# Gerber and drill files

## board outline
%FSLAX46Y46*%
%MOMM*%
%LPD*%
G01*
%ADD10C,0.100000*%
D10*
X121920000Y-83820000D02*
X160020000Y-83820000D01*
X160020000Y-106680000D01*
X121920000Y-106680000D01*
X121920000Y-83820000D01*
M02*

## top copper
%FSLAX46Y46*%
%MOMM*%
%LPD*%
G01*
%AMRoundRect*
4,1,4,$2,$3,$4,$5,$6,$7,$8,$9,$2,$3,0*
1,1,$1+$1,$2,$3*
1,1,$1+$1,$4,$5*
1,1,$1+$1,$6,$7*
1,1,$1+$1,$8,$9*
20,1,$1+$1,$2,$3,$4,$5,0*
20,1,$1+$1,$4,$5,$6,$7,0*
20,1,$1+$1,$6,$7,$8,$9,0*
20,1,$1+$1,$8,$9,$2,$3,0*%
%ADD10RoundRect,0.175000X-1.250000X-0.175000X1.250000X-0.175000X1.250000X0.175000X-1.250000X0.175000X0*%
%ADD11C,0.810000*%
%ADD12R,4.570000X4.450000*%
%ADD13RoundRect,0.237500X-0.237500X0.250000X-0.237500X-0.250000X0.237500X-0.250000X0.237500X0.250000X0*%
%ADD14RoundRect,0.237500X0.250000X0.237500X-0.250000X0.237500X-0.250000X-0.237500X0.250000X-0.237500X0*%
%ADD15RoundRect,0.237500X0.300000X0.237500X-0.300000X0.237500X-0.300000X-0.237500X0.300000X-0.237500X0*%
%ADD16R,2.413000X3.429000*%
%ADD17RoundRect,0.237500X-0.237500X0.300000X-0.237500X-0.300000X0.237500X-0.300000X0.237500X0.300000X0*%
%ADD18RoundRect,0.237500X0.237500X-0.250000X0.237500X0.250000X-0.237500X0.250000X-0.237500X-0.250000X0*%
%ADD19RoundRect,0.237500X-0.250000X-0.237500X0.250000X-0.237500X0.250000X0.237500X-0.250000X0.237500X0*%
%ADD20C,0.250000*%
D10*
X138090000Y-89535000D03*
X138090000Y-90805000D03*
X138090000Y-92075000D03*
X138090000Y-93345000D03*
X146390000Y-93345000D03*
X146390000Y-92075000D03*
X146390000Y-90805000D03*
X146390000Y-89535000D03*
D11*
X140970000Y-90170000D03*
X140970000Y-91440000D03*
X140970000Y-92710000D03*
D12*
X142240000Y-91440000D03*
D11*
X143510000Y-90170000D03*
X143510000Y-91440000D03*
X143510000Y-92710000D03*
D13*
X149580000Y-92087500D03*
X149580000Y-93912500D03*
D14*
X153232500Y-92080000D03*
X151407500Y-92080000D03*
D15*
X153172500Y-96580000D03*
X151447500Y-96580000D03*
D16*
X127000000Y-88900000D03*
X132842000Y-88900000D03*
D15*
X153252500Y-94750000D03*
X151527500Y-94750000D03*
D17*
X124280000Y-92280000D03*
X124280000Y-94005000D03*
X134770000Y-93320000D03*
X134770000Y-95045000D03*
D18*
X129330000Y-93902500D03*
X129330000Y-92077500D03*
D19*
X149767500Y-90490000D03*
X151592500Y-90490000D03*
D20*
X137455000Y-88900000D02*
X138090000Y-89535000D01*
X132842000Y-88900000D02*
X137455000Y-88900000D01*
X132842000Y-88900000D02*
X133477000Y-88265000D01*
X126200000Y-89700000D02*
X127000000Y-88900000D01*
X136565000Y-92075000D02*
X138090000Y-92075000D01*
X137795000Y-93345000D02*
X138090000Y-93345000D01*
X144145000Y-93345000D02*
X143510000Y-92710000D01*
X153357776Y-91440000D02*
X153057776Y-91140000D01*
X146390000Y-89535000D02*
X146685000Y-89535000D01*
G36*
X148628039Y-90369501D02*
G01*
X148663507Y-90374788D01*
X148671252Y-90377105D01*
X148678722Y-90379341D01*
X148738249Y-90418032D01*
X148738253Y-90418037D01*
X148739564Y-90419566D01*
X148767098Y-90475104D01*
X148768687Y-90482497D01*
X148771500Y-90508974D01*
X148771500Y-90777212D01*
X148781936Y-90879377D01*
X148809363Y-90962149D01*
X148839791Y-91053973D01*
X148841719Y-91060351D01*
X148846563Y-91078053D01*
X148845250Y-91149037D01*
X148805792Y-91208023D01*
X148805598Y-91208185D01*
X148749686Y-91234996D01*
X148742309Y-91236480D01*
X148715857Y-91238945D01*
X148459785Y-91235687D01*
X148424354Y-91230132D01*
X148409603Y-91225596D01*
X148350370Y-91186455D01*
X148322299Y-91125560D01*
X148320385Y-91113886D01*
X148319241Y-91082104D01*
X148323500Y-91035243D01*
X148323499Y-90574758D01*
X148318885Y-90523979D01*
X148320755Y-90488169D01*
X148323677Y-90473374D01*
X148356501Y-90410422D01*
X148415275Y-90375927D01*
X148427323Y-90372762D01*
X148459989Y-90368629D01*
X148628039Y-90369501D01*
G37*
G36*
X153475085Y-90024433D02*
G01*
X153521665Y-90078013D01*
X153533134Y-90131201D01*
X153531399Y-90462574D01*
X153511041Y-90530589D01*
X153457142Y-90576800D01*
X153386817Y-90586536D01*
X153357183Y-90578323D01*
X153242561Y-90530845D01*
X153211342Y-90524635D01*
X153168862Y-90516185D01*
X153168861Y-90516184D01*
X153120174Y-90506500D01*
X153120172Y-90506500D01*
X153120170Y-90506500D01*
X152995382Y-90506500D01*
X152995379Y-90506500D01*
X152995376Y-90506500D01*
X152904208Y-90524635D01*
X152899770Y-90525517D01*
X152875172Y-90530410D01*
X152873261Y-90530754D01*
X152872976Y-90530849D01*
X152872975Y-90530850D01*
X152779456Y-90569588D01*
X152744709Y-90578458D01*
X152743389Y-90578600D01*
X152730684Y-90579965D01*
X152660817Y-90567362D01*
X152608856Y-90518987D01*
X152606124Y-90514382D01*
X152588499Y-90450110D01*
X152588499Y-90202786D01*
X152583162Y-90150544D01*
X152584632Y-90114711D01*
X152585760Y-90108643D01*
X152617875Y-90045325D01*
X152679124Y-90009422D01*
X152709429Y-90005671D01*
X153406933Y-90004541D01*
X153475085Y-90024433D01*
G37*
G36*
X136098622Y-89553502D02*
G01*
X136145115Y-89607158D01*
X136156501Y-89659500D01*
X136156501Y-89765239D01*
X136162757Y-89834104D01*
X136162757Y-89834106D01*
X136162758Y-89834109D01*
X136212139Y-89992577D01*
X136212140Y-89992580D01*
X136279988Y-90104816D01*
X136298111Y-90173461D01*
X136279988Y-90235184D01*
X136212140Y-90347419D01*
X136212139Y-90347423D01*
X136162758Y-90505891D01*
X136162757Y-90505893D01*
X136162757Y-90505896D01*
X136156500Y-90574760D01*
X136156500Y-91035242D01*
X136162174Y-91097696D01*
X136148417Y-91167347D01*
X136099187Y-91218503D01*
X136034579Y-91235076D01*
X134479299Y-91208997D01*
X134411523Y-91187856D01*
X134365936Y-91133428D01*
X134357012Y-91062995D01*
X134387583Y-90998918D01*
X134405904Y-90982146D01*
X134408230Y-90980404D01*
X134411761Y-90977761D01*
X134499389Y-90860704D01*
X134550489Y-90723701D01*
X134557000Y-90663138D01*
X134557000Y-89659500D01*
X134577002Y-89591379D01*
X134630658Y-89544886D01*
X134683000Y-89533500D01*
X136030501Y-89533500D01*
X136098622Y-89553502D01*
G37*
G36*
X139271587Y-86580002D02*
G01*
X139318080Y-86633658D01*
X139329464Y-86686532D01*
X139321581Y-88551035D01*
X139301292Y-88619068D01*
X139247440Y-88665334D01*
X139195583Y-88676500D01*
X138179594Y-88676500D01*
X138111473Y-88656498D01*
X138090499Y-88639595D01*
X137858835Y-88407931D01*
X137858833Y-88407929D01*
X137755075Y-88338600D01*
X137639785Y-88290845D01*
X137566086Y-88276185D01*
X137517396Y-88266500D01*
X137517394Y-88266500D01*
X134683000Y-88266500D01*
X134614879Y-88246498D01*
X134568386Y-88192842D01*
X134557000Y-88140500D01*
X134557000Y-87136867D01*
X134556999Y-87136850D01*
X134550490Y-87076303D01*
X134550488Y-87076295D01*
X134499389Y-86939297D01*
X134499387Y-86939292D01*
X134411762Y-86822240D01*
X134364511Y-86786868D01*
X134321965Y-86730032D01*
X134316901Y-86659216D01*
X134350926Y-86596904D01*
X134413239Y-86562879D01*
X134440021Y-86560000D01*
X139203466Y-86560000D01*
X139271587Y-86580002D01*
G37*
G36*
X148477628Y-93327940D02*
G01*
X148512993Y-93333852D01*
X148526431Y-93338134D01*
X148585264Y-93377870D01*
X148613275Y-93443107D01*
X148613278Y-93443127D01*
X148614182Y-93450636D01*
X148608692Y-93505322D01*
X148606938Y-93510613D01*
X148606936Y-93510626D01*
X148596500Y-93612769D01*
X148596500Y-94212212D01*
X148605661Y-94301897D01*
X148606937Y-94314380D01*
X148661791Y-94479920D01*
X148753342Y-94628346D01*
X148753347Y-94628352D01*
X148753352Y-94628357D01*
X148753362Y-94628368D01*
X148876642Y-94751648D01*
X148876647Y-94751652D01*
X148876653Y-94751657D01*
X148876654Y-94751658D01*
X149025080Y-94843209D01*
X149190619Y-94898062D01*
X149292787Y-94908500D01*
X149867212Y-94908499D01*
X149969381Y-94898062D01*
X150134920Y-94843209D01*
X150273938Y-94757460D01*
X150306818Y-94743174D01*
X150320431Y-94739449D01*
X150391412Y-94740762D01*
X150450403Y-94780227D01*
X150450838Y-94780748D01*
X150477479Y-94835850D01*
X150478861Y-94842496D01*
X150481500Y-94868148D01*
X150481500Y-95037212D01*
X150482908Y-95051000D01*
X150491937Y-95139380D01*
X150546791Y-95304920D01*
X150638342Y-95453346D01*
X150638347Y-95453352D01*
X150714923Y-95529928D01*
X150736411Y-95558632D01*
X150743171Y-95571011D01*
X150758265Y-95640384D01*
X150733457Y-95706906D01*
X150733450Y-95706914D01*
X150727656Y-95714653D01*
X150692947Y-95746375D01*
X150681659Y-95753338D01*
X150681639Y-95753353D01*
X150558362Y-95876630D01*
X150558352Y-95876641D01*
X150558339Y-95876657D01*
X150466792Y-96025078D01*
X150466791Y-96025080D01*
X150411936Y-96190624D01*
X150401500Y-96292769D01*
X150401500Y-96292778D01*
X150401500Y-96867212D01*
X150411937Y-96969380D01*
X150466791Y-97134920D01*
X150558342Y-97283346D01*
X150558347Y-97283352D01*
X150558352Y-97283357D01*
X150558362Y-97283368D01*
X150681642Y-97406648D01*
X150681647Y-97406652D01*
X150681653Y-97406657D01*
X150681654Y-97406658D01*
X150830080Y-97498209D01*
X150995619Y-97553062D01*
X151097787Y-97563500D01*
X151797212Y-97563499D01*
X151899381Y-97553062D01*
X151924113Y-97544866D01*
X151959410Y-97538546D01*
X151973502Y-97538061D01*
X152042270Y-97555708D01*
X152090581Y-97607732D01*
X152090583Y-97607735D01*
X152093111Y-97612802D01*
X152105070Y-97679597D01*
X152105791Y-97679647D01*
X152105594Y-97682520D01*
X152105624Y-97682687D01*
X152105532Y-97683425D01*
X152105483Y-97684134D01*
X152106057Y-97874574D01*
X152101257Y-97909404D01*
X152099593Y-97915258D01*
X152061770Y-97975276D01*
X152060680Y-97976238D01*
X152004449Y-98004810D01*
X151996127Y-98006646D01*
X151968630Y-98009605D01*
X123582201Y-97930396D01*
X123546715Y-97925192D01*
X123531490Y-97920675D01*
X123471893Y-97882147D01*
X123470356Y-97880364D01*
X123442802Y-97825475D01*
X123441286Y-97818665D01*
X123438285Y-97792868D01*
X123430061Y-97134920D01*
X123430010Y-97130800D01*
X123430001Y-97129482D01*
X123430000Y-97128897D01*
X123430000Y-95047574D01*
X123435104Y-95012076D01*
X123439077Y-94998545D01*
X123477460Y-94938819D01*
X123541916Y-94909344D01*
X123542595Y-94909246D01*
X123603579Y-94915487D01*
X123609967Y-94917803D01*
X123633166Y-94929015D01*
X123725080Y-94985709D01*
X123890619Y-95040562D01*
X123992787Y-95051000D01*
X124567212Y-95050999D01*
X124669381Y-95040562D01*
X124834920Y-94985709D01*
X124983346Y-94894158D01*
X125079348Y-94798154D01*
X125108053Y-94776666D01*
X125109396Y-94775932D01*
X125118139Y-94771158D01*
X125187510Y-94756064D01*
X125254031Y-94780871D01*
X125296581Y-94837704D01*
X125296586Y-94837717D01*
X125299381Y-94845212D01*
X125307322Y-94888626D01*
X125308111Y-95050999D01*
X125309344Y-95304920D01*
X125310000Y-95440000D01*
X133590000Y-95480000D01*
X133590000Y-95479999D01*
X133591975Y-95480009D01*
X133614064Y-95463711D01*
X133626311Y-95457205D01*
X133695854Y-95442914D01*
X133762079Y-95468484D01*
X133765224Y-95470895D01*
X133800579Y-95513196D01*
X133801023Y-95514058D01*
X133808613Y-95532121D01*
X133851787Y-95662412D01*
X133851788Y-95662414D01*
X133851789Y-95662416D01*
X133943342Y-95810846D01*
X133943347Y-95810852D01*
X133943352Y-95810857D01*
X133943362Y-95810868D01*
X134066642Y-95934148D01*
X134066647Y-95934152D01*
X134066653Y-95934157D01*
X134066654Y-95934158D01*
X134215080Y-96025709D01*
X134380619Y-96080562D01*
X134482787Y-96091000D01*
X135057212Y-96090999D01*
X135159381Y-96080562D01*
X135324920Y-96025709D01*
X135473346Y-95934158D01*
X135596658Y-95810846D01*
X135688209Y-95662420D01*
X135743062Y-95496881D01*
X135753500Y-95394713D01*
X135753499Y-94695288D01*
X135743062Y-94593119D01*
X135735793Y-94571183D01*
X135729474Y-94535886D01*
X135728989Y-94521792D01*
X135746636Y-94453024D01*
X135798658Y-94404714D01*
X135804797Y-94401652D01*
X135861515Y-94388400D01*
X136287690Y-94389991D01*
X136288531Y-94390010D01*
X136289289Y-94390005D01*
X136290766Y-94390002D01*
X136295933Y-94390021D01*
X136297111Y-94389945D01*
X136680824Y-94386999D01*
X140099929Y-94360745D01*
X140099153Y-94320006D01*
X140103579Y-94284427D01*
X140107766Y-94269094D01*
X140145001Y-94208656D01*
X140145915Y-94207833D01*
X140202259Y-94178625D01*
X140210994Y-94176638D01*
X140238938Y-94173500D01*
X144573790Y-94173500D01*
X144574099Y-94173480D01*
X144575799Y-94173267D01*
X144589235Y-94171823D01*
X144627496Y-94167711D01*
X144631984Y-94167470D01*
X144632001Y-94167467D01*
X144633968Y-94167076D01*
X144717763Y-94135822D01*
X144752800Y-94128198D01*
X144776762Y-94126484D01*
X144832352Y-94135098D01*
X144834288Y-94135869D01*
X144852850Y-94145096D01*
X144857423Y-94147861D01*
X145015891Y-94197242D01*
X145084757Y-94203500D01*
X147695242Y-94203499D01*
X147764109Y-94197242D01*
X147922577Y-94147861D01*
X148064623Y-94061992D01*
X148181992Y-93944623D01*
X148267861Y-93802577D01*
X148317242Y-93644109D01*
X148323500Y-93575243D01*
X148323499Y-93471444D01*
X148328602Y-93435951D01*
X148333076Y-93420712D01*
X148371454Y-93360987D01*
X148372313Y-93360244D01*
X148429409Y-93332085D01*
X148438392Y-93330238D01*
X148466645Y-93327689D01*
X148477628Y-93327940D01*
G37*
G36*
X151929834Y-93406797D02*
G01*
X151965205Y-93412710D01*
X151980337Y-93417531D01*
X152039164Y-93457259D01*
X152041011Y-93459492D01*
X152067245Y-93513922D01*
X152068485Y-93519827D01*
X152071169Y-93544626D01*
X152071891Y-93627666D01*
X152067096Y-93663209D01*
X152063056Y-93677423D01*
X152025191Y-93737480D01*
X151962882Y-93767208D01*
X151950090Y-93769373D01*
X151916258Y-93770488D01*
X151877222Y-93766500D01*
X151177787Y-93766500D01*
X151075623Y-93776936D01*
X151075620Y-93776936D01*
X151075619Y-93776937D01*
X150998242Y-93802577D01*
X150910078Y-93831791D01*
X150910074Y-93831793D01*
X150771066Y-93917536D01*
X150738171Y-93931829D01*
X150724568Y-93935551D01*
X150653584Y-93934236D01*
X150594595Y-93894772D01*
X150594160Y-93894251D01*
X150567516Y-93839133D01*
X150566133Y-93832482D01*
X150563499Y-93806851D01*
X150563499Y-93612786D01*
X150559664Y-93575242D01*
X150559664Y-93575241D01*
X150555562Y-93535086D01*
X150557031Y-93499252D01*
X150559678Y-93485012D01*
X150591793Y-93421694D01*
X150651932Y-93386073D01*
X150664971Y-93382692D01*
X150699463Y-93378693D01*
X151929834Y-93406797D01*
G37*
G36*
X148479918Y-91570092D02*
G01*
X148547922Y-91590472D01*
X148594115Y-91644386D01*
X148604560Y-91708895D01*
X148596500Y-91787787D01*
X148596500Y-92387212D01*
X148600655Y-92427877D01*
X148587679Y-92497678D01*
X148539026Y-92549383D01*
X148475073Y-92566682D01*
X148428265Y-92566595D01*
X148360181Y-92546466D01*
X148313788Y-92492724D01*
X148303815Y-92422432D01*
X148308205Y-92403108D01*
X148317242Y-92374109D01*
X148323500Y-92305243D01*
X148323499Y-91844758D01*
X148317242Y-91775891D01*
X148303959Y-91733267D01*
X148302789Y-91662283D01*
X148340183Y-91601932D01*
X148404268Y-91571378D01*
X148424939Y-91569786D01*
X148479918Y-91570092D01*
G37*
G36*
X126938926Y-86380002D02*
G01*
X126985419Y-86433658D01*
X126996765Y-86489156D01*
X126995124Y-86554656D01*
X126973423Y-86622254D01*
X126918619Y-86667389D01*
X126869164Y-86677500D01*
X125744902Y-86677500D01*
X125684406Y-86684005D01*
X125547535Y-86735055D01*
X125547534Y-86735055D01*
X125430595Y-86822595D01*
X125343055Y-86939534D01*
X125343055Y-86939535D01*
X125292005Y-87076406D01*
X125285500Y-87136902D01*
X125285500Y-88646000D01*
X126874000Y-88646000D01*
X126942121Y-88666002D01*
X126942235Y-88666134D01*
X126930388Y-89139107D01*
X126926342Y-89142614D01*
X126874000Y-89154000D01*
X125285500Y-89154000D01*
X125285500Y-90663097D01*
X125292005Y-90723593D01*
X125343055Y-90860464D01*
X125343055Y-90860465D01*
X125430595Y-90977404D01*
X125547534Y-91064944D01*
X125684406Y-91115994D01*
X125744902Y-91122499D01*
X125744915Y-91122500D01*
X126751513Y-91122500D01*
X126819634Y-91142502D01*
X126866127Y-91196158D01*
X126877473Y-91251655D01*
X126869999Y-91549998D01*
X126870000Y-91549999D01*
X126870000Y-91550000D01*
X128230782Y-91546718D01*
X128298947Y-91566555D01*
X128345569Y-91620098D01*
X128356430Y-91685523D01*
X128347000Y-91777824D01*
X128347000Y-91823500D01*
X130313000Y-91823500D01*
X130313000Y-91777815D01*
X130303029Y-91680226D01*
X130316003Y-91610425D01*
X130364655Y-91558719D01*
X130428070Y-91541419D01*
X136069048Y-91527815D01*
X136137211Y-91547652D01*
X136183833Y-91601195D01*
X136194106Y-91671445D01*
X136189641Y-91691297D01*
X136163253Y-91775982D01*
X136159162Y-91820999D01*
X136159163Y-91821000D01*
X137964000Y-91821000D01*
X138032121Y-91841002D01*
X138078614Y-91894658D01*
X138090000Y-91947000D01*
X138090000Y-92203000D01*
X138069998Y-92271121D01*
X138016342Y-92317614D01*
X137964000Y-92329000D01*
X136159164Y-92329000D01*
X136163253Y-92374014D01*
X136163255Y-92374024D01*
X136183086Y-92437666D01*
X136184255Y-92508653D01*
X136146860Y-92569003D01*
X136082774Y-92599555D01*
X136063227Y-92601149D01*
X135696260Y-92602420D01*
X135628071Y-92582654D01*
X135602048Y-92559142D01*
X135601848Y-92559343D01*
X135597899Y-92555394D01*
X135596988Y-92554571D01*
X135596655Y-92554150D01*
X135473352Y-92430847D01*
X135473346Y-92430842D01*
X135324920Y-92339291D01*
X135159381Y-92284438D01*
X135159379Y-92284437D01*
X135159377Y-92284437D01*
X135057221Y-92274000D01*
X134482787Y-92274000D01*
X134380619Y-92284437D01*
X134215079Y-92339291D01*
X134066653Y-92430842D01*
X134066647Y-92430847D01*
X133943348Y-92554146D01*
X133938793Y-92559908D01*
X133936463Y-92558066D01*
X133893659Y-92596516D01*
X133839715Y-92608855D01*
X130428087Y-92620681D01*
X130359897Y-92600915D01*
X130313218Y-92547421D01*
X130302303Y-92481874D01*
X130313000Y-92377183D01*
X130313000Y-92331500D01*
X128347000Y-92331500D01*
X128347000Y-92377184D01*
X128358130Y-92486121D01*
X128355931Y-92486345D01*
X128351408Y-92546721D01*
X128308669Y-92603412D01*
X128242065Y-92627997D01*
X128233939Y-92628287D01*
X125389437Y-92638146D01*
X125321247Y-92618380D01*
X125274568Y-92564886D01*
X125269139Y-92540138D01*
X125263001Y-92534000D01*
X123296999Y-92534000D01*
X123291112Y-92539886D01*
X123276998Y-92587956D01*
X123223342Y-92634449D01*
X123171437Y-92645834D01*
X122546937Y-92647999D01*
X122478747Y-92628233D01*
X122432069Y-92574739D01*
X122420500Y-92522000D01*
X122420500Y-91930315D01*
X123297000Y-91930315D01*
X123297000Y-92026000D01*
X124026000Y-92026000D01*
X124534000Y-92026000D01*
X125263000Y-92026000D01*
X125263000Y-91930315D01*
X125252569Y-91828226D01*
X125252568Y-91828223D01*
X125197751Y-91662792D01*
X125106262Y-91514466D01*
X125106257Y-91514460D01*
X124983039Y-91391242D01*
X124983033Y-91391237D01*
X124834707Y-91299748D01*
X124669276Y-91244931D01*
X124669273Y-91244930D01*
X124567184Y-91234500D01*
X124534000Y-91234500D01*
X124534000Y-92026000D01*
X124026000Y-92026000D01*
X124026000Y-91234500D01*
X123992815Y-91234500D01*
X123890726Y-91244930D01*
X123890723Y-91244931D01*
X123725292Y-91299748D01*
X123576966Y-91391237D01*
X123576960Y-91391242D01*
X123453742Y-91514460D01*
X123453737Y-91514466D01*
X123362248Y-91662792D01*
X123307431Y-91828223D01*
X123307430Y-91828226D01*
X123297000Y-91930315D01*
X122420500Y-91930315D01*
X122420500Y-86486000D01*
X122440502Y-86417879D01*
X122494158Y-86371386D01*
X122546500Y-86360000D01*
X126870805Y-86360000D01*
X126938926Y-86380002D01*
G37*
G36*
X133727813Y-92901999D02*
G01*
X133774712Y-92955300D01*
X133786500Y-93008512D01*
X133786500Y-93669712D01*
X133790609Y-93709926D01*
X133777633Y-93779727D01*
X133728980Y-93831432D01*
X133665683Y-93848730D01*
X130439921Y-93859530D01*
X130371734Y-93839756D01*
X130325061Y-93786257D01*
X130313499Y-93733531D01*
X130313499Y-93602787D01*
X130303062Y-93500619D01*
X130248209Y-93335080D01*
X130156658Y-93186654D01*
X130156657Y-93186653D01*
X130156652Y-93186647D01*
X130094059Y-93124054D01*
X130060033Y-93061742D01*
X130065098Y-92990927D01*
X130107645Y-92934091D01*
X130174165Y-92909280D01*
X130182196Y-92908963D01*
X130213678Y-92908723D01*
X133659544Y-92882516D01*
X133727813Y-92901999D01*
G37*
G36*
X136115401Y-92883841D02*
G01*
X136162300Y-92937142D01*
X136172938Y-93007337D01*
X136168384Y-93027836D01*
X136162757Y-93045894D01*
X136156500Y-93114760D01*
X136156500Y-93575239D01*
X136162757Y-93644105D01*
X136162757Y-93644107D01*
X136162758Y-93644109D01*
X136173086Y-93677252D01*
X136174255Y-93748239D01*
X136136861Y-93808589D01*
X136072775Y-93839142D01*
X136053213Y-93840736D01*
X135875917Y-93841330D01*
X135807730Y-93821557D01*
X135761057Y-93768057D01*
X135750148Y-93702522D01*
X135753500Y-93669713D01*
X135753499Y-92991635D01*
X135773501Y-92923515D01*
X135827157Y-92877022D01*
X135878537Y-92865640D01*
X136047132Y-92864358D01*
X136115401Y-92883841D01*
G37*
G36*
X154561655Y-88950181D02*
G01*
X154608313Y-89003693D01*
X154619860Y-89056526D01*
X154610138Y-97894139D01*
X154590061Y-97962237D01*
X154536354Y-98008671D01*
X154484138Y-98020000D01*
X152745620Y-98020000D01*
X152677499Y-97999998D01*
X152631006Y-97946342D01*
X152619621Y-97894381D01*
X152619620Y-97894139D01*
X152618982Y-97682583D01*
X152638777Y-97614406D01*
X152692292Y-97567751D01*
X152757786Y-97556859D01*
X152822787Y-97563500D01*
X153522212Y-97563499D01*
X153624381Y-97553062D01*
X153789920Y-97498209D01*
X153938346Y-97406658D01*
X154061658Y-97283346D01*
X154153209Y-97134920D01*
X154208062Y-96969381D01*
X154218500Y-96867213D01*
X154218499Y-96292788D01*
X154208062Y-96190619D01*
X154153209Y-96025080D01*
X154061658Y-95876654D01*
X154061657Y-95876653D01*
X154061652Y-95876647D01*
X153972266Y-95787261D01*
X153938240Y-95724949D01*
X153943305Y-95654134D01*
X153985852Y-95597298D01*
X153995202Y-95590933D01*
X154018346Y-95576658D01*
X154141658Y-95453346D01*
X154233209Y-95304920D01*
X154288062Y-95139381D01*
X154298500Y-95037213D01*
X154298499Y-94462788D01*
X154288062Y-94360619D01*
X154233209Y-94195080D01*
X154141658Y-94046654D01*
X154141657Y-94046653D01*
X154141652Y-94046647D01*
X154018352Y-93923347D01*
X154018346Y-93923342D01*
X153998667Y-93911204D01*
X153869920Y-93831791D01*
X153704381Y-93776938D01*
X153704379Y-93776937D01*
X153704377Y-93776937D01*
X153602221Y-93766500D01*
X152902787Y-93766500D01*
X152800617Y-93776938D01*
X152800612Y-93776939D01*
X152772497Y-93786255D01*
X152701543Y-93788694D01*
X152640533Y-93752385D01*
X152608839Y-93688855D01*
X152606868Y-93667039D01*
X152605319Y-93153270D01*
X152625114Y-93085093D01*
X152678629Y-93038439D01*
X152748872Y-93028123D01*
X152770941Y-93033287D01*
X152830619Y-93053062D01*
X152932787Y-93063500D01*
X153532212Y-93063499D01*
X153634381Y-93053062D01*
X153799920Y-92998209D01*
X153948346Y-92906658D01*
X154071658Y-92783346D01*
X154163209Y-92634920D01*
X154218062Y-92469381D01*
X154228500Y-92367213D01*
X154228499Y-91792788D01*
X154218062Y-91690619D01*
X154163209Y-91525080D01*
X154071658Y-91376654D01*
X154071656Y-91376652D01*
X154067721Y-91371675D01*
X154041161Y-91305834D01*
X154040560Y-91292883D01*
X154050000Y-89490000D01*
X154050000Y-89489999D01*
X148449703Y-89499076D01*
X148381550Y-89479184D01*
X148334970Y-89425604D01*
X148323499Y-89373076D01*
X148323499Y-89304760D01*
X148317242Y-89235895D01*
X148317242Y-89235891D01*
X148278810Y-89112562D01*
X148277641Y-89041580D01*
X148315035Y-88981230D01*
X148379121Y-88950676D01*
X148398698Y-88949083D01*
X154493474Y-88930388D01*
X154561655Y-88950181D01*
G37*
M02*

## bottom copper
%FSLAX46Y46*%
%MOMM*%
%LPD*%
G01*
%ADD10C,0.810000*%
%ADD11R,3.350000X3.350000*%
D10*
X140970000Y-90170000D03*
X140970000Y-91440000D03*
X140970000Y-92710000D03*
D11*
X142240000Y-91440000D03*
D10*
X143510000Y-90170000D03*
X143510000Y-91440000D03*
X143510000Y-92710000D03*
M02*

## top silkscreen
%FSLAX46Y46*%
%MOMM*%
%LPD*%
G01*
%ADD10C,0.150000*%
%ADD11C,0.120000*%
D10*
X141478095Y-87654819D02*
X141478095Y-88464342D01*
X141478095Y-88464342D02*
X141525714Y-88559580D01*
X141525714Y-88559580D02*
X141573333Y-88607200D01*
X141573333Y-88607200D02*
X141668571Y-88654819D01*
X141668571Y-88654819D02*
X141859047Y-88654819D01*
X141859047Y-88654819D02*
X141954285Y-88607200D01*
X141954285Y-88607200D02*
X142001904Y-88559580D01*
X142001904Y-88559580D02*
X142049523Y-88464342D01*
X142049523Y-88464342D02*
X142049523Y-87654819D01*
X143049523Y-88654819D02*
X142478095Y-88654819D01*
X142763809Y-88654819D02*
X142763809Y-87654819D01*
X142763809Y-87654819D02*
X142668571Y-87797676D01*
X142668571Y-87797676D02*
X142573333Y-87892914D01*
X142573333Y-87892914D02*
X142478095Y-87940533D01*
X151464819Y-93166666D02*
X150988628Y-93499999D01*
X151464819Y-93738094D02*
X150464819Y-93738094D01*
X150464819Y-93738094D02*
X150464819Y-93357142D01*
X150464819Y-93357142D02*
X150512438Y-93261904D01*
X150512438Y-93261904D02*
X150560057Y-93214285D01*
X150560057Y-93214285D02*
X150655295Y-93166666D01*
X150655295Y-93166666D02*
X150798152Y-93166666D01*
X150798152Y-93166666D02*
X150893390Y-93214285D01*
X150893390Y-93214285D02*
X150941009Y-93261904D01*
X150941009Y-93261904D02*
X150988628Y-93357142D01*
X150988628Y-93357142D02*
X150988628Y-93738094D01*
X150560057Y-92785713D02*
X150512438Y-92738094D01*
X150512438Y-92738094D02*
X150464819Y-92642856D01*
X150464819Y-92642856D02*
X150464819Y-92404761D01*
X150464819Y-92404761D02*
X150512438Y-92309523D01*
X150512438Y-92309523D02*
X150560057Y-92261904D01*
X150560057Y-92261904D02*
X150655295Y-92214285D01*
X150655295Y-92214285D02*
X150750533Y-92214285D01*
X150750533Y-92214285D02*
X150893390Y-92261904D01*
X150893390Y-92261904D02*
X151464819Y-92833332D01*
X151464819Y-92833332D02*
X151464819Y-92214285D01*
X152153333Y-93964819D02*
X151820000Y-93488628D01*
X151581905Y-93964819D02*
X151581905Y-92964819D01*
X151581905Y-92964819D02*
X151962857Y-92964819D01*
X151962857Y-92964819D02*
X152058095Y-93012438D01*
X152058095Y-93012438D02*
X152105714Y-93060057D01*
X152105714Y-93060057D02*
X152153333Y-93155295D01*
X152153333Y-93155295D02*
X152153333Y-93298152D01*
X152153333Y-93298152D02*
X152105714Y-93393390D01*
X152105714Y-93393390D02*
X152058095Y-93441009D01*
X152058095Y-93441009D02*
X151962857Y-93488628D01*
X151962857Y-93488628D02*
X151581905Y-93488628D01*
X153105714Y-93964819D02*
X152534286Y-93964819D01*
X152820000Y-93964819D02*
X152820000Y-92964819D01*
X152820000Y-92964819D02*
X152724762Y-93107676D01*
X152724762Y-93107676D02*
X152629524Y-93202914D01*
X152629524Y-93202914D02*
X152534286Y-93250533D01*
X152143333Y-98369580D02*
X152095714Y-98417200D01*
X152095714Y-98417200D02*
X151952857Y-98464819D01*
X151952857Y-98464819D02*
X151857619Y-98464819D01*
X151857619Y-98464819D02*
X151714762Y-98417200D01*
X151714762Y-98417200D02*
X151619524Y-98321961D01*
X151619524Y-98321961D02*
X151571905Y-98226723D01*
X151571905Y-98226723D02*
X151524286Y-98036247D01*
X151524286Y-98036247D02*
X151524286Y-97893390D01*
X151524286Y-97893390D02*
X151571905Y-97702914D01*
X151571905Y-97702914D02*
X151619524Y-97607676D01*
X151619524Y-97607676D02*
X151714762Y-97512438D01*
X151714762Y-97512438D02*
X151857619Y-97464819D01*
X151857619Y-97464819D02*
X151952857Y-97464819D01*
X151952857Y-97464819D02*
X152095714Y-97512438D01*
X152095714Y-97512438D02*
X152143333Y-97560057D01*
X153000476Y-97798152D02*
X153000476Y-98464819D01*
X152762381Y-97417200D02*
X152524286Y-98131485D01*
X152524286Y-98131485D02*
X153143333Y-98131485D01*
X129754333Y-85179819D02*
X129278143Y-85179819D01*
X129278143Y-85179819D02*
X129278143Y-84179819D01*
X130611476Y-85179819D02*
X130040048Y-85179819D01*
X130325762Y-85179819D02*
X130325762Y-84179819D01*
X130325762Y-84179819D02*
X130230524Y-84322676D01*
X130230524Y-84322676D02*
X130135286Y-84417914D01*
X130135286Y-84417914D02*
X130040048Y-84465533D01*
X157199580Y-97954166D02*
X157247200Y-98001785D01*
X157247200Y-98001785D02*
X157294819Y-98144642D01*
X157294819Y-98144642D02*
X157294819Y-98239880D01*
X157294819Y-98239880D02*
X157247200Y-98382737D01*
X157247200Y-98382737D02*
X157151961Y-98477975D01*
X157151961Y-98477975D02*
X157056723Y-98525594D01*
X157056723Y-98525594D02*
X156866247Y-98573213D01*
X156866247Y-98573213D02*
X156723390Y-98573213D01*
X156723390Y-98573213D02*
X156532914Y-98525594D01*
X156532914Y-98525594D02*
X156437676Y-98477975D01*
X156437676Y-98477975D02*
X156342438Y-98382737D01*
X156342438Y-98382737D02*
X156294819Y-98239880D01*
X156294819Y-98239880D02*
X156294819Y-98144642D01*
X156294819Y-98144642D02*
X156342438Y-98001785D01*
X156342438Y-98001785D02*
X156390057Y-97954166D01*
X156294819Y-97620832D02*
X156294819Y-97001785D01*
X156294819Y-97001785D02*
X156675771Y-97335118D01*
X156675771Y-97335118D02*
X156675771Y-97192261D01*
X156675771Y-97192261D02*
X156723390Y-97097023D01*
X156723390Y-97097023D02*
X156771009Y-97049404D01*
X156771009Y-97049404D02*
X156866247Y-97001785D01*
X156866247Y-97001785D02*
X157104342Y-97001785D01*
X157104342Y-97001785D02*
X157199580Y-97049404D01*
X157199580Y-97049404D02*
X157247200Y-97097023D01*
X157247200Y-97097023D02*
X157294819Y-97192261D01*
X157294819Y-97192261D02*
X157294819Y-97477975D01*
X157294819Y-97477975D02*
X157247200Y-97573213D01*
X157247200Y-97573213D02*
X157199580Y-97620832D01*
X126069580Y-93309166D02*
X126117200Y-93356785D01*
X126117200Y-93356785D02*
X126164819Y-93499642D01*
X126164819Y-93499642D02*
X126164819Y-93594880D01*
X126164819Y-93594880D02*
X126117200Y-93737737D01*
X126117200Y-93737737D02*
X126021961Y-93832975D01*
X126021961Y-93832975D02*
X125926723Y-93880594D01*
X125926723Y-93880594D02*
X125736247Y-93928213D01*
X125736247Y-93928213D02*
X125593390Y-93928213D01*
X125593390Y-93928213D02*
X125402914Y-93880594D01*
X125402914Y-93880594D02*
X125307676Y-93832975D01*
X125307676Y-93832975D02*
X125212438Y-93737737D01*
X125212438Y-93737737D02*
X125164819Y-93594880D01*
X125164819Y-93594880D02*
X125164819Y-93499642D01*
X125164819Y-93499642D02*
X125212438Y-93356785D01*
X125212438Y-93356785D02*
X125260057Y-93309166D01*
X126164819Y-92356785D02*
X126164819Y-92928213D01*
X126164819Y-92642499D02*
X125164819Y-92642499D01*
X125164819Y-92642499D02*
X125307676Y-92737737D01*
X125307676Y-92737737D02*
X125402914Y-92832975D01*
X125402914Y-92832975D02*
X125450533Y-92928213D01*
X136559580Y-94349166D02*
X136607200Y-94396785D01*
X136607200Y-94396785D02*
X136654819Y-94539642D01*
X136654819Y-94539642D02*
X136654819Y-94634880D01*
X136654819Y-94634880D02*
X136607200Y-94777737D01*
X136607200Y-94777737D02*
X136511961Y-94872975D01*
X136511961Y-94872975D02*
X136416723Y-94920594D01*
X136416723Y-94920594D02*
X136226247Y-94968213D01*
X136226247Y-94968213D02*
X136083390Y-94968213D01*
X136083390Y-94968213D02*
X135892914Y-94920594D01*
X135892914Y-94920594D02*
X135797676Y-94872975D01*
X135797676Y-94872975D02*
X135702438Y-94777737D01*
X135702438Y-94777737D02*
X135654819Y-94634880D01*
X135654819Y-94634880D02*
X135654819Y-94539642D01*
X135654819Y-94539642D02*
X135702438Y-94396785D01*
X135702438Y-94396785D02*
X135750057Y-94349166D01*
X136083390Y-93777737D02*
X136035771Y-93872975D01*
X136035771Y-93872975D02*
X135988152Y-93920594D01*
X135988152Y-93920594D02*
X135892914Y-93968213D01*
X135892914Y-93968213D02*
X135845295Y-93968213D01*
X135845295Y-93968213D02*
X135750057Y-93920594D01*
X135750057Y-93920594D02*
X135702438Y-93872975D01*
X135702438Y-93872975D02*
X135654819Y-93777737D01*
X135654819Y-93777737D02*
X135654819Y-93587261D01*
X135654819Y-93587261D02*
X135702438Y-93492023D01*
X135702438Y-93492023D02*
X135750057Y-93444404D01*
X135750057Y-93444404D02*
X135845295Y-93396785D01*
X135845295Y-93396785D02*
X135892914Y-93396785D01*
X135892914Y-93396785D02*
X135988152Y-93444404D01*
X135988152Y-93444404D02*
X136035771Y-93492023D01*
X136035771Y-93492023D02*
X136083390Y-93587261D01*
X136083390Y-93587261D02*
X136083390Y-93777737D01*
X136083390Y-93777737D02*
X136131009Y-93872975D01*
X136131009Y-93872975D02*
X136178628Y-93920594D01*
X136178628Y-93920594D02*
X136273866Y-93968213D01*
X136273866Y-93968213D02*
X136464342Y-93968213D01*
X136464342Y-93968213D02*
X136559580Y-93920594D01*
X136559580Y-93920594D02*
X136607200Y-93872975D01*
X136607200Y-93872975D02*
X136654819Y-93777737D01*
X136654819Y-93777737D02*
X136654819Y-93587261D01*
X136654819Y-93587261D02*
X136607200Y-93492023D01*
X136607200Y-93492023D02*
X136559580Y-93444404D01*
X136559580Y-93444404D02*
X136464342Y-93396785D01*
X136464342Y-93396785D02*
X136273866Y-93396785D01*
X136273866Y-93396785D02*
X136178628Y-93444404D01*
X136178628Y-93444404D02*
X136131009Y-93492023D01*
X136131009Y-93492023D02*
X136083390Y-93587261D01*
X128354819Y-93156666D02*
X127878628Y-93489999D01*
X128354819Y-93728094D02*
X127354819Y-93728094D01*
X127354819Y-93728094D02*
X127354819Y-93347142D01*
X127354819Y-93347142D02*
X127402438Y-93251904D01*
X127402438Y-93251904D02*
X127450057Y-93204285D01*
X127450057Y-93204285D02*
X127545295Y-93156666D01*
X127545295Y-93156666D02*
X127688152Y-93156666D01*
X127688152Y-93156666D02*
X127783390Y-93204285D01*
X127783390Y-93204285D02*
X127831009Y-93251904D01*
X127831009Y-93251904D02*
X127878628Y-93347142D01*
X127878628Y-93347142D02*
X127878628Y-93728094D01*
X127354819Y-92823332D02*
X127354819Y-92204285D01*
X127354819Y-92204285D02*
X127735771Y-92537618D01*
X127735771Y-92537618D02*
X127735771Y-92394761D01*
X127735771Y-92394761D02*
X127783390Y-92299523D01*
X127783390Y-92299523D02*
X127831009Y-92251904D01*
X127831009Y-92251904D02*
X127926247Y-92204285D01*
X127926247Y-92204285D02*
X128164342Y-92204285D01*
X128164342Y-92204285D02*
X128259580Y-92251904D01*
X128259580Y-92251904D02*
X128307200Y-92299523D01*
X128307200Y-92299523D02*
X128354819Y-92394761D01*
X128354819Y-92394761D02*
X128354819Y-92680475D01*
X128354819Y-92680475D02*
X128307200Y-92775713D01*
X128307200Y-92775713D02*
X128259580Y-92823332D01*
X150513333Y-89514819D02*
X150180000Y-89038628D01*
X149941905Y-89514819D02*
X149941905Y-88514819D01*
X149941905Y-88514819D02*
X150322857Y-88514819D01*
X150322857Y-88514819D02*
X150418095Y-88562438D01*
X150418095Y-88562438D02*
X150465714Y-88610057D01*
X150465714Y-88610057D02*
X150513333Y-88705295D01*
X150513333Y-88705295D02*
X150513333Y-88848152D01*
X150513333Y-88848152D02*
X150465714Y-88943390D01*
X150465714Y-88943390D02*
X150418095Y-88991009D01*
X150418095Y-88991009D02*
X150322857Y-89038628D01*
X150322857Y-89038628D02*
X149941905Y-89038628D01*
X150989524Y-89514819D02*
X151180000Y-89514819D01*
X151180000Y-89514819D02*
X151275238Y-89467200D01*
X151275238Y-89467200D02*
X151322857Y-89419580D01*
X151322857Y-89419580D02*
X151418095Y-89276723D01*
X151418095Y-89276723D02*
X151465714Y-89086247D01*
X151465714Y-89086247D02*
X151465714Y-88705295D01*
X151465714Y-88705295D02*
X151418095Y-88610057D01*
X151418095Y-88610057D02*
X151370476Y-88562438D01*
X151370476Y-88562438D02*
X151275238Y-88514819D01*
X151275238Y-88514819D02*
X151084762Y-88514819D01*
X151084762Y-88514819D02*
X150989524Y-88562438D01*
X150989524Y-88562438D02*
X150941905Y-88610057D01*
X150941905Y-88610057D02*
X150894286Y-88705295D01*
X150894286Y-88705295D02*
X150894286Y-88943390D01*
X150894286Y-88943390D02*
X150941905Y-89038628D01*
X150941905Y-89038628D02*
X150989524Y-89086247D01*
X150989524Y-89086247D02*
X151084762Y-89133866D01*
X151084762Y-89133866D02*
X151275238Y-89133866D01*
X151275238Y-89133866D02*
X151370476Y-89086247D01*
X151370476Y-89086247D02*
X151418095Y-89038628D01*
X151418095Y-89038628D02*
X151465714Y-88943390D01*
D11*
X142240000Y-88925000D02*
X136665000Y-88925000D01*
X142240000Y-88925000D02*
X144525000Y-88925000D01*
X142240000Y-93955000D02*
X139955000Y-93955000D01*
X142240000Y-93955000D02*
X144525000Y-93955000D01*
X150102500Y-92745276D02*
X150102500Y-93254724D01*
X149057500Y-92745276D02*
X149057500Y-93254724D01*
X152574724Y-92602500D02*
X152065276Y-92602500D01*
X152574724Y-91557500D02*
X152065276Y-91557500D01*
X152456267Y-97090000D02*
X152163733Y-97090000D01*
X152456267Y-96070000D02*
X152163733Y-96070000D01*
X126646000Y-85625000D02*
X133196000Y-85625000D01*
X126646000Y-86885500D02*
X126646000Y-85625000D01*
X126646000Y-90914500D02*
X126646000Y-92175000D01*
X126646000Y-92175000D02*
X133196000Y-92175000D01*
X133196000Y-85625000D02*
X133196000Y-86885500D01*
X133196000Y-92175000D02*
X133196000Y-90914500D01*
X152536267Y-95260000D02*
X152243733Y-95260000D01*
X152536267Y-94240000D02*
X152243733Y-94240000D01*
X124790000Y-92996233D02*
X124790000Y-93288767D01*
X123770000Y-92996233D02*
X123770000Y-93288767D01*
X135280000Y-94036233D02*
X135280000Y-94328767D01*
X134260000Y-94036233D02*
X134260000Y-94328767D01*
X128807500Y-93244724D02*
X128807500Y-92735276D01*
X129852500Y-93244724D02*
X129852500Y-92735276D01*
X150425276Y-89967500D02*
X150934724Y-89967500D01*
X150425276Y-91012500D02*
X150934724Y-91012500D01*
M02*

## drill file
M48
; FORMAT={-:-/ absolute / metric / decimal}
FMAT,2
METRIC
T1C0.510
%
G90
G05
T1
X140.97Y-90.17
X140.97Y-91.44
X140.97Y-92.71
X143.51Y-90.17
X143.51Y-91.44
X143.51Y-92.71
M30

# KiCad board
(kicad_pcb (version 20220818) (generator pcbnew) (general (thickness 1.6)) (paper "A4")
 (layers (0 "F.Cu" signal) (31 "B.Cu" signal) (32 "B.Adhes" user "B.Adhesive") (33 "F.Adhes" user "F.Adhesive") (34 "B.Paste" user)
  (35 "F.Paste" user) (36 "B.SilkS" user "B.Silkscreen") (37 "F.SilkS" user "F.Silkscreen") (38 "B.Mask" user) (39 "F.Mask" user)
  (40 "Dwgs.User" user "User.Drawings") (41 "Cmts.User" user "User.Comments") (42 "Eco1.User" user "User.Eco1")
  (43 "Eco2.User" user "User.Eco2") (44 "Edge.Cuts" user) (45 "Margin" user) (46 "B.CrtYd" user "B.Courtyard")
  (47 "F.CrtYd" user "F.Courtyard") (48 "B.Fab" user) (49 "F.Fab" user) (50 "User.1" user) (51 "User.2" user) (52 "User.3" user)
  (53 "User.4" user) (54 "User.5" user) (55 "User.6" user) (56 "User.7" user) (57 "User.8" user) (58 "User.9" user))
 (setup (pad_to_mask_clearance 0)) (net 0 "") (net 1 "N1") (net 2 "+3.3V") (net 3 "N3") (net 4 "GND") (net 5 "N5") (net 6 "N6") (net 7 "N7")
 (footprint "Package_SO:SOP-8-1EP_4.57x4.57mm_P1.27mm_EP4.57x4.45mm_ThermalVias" (layer "F.Cu") (at 142.24 91.44)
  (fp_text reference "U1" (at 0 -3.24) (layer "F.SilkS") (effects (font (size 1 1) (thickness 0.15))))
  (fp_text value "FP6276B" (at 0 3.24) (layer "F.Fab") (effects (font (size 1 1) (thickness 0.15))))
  (fp_line (start 0 -2.515) (end -5.575 -2.515) (stroke (width 0.12) (type solid)) (layer "F.SilkS"))
  (fp_line (start 0 -2.515) (end 2.285 -2.515) (stroke (width 0.12) (type solid)) (layer "F.SilkS"))
  (fp_line (start 0 2.515) (end -2.285 2.515) (stroke (width 0.12) (type solid)) (layer "F.SilkS"))
  (fp_line (start 0 2.515) (end 2.285 2.515) (stroke (width 0.12) (type solid)) (layer "F.SilkS"))
  (pad "" smd roundrect (at -1.14 -1.11) (size 1.91 1.86) (layers "F.Paste") (roundrect_rratio 0.134409))
  (pad "" smd roundrect (at -1.14 1.11) (size 1.91 1.86) (layers "F.Paste") (roundrect_rratio 0.134409))
  (pad "" smd roundrect (at 1.14 -1.11) (size 1.91 1.86) (layers "F.Paste") (roundrect_rratio 0.134409))
  (pad "" smd roundrect (at 1.14 1.11) (size 1.91 1.86) (layers "F.Paste") (roundrect_rratio 0.134409))
  (pad "1" smd roundrect (at -4.15 -1.905) (size 2.85 0.7) (layers "F.Cu" "F.Paste" "F.Mask") (roundrect_rratio 0.25) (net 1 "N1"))
  (pad "2" smd roundrect (at -4.15 -0.635) (size 2.85 0.7) (layers "F.Cu" "F.Paste" "F.Mask") (roundrect_rratio 0.25) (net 1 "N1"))
  (pad "3" smd roundrect (at -4.15 0.635) (size 2.85 0.7) (layers "F.Cu" "F.Paste" "F.Mask") (roundrect_rratio 0.25) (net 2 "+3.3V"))
  (pad "4" smd roundrect (at -4.15 1.905) (size 2.85 0.7) (layers "F.Cu" "F.Paste" "F.Mask") (roundrect_rratio 0.25) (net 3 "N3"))
  (pad "5" smd roundrect (at 4.15 1.905) (size 2.85 0.7) (layers "F.Cu" "F.Paste" "F.Mask") (roundrect_rratio 0.25) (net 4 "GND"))
  (pad "6" smd roundrect (at 4.15 0.635) (size 2.85 0.7) (layers "F.Cu" "F.Paste" "F.Mask") (roundrect_rratio 0.25) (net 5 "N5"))
  (pad "7" smd roundrect (at 4.15 -0.635) (size 2.85 0.7) (layers "F.Cu" "F.Paste" "F.Mask") (roundrect_rratio 0.25) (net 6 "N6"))
  (pad "8" smd roundrect (at 4.15 -1.905) (size 2.85 0.7) (layers "F.Cu" "F.Paste" "F.Mask") (roundrect_rratio 0.25) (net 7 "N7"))
  (pad "9" thru_hole circle (at -1.27 -1.27) (size 0.81 0.81) (drill 0.51) (layers *.Cu) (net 4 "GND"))
  (pad "9" thru_hole circle (at -1.27 0) (size 0.81 0.81) (drill 0.51) (layers *.Cu) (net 4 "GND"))
  (pad "9" thru_hole circle (at -1.27 1.27) (size 0.81 0.81) (drill 0.51) (layers *.Cu) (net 4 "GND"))
  (pad "9" smd rect (at 0 0) (size 3.35 3.35) (layers "B.Cu") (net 4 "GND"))
  (pad "9" smd rect (at 0 0) (size 4.57 4.45) (layers "F.Cu" "F.Mask") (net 4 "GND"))
  (pad "9" thru_hole circle (at 1.27 -1.27) (size 0.81 0.81) (drill 0.51) (layers *.Cu) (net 4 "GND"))
  (pad "9" thru_hole circle (at 1.27 0) (size 0.81 0.81) (drill 0.51) (layers *.Cu) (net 4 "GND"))
  (pad "9" thru_hole circle (at 1.27 1.27) (size 0.81 0.81) (drill 0.51) (layers *.Cu) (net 4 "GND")))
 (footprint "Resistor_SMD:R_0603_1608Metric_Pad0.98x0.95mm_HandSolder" (layer "F.Cu") (at 149.58 93 -90)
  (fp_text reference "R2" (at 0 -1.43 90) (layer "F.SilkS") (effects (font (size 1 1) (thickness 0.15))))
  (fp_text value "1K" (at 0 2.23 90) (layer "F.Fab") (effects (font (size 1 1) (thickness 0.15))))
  (fp_line (start -0.254724 -0.5225) (end 0.254724 -0.5225) (stroke (width 0.12) (type solid)) (layer "F.SilkS"))
  (fp_line (start -0.254724 0.5225) (end 0.254724 0.5225) (stroke (width 0.12) (type solid)) (layer "F.SilkS"))
  (pad "1" smd roundrect (at -0.9125 0 270) (size 0.975 0.95) (layers "F.Cu" "F.Paste" "F.Mask") (roundrect_rratio 0.25) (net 5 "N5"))
  (pad "2" smd roundrect (at 0.9125 0 270) (size 0.975 0.95) (layers "F.Cu" "F.Paste" "F.Mask") (roundrect_rratio 0.25) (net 4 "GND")))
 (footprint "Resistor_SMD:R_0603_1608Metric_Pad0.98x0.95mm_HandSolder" (layer "F.Cu") (at 152.32 92.08 180)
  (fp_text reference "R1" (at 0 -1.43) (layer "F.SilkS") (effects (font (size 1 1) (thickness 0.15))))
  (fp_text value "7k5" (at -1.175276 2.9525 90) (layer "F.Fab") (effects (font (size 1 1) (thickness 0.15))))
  (fp_line (start -0.254724 -0.5225) (end 0.254724 -0.5225) (stroke (width 0.12) (type solid)) (layer "F.SilkS"))
  (fp_line (start -0.254724 0.5225) (end 0.254724 0.5225) (stroke (width 0.12) (type solid)) (layer "F.SilkS"))
  (pad "1" smd roundrect (at -0.9125 0 180) (size 0.975 0.95) (layers "F.Cu" "F.Paste" "F.Mask") (roundrect_rratio 0.25) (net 7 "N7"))
  (pad "2" smd roundrect (at 0.9125 0 180) (size 0.975 0.95) (layers "F.Cu" "F.Paste" "F.Mask") (roundrect_rratio 0.25) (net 5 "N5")))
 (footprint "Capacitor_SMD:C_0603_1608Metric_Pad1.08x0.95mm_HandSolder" (layer "F.Cu") (at 152.31 96.58 180)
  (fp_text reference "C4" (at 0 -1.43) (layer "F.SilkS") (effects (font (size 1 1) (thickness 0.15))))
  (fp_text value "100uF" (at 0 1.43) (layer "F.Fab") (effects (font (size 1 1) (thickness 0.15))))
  (fp_line (start -0.146267 -0.51) (end 0.146267 -0.51) (stroke (width 0.12) (type solid)) (layer "F.SilkS"))
  (fp_line (start -0.146267 0.51) (end 0.146267 0.51) (stroke (width 0.12) (type solid)) (layer "F.SilkS"))
  (pad "1" smd roundrect (at -0.8625 0 180) (size 1.075 0.95) (layers "F.Cu" "F.Paste" "F.Mask") (roundrect_rratio 0.25) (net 7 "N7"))
  (pad "2" smd roundrect (at 0.8625 0 180) (size 1.075 0.95) (layers "F.Cu" "F.Paste" "F.Mask") (roundrect_rratio 0.25) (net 4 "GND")))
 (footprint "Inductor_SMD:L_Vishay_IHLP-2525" (layer "F.Cu") (at 129.921 88.9)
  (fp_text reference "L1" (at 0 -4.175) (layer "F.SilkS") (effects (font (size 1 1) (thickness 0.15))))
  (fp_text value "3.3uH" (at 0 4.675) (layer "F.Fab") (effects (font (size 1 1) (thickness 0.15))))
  (fp_line (start -3.275 -3.275) (end 3.275 -3.275) (stroke (width 0.12) (type solid)) (layer "F.SilkS"))
  (fp_line (start -3.275 -2.0145) (end -3.275 -3.275) (stroke (width 0.12) (type solid)) (layer "F.SilkS"))
  (fp_line (start -3.275 2.0145) (end -3.275 3.275) (stroke (width 0.12) (type solid)) (layer "F.SilkS"))
  (fp_line (start -3.275 3.275) (end 3.275 3.275) (stroke (width 0.12) (type solid)) (layer "F.SilkS"))
  (fp_line (start 3.275 -3.275) (end 3.275 -2.0145) (stroke (width 0.12) (type solid)) (layer "F.SilkS"))
  (fp_line (start 3.275 3.275) (end 3.275 2.0145) (stroke (width 0.12) (type solid)) (layer "F.SilkS"))
  (pad "1" smd rect (at -2.921 0) (size 2.413 3.429) (layers "F.Cu" "F.Paste" "F.Mask") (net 2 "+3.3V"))
  (pad "2" smd rect (at 2.921 0) (size 2.413 3.429) (layers "F.Cu" "F.Paste" "F.Mask") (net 1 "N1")))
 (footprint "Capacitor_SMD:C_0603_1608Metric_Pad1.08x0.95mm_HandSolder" (layer "F.Cu") (at 152.39 94.75 180)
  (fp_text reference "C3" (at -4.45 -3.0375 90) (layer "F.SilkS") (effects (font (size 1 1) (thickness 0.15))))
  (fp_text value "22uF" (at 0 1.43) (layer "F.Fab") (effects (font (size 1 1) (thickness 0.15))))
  (fp_line (start -0.146267 -0.51) (end 0.146267 -0.51) (stroke (width 0.12) (type solid)) (layer "F.SilkS"))
  (fp_line (start -0.146267 0.51) (end 0.146267 0.51) (stroke (width 0.12) (type solid)) (layer "F.SilkS"))
  (pad "1" smd roundrect (at -0.8625 0 180) (size 1.075 0.95) (layers "F.Cu" "F.Paste" "F.Mask") (roundrect_rratio 0.25) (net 7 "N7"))
  (pad "2" smd roundrect (at 0.8625 0 180) (size 1.075 0.95) (layers "F.Cu" "F.Paste" "F.Mask") (roundrect_rratio 0.25) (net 4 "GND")))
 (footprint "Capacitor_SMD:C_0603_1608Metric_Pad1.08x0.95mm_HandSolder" (layer "F.Cu") (at 124.28 93.1425 -90)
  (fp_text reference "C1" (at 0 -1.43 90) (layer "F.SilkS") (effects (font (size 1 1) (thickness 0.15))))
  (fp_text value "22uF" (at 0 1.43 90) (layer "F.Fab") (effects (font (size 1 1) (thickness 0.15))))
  (fp_line (start -0.146267 -0.51) (end 0.146267 -0.51) (stroke (width 0.12) (type solid)) (layer "F.SilkS"))
  (fp_line (start -0.146267 0.51) (end 0.146267 0.51) (stroke (width 0.12) (type solid)) (layer "F.SilkS"))
  (pad "1" smd roundrect (at -0.8625 0 270) (size 1.075 0.95) (layers "F.Cu" "F.Paste" "F.Mask") (roundrect_rratio 0.25) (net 2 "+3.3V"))
  (pad "2" smd roundrect (at 0.8625 0 270) (size 1.075 0.95) (layers "F.Cu" "F.Paste" "F.Mask") (roundrect_rratio 0.25) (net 4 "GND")))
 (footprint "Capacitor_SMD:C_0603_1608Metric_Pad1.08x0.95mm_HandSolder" (layer "F.Cu") (at 134.77 94.1825 -90)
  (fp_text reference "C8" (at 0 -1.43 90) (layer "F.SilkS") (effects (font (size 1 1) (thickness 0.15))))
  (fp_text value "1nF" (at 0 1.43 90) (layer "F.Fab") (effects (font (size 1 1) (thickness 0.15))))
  (fp_line (start -0.146267 -0.51) (end 0.146267 -0.51) (stroke (width 0.12) (type solid)) (layer "F.SilkS"))
  (fp_line (start -0.146267 0.51) (end 0.146267 0.51) (stroke (width 0.12) (type solid)) (layer "F.SilkS"))
  (pad "1" smd roundrect (at -0.8625 0 270) (size 1.075 0.95) (layers "F.Cu" "F.Paste" "F.Mask") (roundrect_rratio 0.25) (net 3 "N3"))
  (pad "2" smd roundrect (at 0.8625 0 270) (size 1.075 0.95) (layers "F.Cu" "F.Paste" "F.Mask") (roundrect_rratio 0.25) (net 4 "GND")))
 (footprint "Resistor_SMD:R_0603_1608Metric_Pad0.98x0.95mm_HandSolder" (layer "F.Cu") (at 129.33 92.99 90)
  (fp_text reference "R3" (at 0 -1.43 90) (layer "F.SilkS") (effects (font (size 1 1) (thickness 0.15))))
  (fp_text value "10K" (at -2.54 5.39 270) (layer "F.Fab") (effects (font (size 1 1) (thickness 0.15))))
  (fp_line (start -0.254724 -0.5225) (end 0.254724 -0.5225) (stroke (width 0.12) (type solid)) (layer "F.SilkS"))
  (fp_line (start -0.254724 0.5225) (end 0.254724 0.5225) (stroke (width 0.12) (type solid)) (layer "F.SilkS"))
  (pad "1" smd roundrect (at -0.9125 0 90) (size 0.975 0.95) (layers "F.Cu" "F.Paste" "F.Mask") (roundrect_rratio 0.25) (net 3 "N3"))
  (pad "2" smd roundrect (at 0.9125 0 90) (size 0.975 0.95) (layers "F.Cu" "F.Paste" "F.Mask") (roundrect_rratio 0.25) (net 2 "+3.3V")))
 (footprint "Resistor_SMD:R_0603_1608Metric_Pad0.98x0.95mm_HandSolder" (layer "F.Cu") (at 150.68 90.49)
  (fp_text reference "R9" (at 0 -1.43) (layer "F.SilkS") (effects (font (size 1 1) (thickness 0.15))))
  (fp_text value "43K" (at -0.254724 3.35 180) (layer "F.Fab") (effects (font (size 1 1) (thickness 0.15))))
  (fp_line (start -0.254724 -0.5225) (end 0.254724 -0.5225) (stroke (width 0.12) (type solid)) (layer "F.SilkS"))
  (fp_line (start -0.254724 0.5225) (end 0.254724 0.5225) (stroke (width 0.12) (type solid)) (layer "F.SilkS"))
  (pad "1" smd roundrect (at -0.9125 0) (size 0.975 0.95) (layers "F.Cu" "F.Paste" "F.Mask") (roundrect_rratio 0.25) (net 6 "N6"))
  (pad "2" smd roundrect (at 0.9125 0) (size 0.975 0.95) (layers "F.Cu" "F.Paste" "F.Mask") (roundrect_rratio 0.25) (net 4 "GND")))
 (gr_rect (start 121.92 83.82) (end 160.02 106.68) (stroke (width 0.1) (type default)) (fill none) (layer "Edge.Cuts"))
 (segment (start 137.455 88.9) (end 138.09 89.535) (width 0.25) (layer "F.Cu") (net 1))
 (segment (start 132.842 88.9) (end 137.455 88.9) (width 0.25) (layer "F.Cu") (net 1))
 (segment (start 132.842 88.9) (end 133.477 88.265) (width 0.25) (layer "F.Cu") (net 1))
 (segment (start 126.2 89.7) (end 127 88.9) (width 0.25) (layer "F.Cu") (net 2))
 (segment (start 136.565 92.075) (end 138.09 92.075) (width 0.25) (layer "F.Cu") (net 2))
 (segment (start 137.795 93.345) (end 138.09 93.345) (width 0.25) (layer "F.Cu") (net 3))
 (segment (start 144.145 93.345) (end 143.51 92.71) (width 0.25) (layer "F.Cu") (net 4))
 (segment (start 153.357776 91.44) (end 153.057776 91.14) (width 0.25) (layer "F.Cu") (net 7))
 (segment (start 146.39 89.535) (end 146.685 89.535) (width 0.25) (layer "F.Cu") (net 7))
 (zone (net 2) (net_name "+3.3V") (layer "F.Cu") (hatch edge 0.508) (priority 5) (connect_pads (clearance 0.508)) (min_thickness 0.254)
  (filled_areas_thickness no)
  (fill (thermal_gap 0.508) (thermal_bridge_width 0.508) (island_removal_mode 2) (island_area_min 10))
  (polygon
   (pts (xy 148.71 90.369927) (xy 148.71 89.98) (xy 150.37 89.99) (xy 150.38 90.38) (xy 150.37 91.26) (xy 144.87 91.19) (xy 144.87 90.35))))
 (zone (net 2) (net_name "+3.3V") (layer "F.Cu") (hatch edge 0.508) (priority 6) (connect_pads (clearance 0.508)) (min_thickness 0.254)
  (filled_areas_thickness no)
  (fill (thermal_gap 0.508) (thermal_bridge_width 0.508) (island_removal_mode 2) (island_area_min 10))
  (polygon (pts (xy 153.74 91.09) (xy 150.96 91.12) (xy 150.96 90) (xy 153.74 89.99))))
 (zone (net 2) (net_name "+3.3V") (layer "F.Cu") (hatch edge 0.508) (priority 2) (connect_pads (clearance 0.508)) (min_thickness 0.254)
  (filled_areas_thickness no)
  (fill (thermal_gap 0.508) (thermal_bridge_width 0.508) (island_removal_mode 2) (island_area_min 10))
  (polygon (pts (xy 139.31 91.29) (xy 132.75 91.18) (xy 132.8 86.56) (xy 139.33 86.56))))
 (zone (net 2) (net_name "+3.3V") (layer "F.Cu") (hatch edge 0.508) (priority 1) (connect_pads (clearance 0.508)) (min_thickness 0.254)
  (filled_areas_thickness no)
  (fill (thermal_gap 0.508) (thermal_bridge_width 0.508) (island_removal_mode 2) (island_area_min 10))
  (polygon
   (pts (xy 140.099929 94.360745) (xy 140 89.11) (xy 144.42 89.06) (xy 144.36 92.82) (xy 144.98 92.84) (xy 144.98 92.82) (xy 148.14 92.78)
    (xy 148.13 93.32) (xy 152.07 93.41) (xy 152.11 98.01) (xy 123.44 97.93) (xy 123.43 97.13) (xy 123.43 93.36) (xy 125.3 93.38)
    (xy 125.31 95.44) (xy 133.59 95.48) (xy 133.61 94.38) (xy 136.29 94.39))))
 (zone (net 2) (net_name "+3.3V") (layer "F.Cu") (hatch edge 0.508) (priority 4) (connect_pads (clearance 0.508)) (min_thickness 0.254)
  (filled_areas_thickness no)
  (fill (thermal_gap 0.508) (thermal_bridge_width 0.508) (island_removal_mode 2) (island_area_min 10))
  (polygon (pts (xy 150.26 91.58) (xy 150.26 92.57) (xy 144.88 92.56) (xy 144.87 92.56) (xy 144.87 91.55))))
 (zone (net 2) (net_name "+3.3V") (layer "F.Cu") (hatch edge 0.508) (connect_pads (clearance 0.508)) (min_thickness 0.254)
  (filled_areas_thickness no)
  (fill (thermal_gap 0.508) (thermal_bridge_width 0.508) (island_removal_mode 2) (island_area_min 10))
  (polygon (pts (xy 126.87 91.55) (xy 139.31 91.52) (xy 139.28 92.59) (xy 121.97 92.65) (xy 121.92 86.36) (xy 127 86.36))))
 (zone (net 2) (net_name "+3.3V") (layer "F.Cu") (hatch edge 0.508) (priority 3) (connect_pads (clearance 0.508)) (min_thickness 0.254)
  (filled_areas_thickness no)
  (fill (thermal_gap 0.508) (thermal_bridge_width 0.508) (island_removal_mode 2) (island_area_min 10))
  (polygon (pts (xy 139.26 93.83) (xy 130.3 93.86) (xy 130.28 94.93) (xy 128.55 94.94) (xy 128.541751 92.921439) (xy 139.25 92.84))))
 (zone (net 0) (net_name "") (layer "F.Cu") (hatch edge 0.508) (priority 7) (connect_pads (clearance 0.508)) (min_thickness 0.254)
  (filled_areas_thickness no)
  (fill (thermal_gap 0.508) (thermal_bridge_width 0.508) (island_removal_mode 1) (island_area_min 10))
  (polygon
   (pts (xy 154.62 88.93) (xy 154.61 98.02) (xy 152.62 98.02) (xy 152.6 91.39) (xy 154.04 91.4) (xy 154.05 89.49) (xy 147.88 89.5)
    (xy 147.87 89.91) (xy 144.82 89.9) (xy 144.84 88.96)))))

